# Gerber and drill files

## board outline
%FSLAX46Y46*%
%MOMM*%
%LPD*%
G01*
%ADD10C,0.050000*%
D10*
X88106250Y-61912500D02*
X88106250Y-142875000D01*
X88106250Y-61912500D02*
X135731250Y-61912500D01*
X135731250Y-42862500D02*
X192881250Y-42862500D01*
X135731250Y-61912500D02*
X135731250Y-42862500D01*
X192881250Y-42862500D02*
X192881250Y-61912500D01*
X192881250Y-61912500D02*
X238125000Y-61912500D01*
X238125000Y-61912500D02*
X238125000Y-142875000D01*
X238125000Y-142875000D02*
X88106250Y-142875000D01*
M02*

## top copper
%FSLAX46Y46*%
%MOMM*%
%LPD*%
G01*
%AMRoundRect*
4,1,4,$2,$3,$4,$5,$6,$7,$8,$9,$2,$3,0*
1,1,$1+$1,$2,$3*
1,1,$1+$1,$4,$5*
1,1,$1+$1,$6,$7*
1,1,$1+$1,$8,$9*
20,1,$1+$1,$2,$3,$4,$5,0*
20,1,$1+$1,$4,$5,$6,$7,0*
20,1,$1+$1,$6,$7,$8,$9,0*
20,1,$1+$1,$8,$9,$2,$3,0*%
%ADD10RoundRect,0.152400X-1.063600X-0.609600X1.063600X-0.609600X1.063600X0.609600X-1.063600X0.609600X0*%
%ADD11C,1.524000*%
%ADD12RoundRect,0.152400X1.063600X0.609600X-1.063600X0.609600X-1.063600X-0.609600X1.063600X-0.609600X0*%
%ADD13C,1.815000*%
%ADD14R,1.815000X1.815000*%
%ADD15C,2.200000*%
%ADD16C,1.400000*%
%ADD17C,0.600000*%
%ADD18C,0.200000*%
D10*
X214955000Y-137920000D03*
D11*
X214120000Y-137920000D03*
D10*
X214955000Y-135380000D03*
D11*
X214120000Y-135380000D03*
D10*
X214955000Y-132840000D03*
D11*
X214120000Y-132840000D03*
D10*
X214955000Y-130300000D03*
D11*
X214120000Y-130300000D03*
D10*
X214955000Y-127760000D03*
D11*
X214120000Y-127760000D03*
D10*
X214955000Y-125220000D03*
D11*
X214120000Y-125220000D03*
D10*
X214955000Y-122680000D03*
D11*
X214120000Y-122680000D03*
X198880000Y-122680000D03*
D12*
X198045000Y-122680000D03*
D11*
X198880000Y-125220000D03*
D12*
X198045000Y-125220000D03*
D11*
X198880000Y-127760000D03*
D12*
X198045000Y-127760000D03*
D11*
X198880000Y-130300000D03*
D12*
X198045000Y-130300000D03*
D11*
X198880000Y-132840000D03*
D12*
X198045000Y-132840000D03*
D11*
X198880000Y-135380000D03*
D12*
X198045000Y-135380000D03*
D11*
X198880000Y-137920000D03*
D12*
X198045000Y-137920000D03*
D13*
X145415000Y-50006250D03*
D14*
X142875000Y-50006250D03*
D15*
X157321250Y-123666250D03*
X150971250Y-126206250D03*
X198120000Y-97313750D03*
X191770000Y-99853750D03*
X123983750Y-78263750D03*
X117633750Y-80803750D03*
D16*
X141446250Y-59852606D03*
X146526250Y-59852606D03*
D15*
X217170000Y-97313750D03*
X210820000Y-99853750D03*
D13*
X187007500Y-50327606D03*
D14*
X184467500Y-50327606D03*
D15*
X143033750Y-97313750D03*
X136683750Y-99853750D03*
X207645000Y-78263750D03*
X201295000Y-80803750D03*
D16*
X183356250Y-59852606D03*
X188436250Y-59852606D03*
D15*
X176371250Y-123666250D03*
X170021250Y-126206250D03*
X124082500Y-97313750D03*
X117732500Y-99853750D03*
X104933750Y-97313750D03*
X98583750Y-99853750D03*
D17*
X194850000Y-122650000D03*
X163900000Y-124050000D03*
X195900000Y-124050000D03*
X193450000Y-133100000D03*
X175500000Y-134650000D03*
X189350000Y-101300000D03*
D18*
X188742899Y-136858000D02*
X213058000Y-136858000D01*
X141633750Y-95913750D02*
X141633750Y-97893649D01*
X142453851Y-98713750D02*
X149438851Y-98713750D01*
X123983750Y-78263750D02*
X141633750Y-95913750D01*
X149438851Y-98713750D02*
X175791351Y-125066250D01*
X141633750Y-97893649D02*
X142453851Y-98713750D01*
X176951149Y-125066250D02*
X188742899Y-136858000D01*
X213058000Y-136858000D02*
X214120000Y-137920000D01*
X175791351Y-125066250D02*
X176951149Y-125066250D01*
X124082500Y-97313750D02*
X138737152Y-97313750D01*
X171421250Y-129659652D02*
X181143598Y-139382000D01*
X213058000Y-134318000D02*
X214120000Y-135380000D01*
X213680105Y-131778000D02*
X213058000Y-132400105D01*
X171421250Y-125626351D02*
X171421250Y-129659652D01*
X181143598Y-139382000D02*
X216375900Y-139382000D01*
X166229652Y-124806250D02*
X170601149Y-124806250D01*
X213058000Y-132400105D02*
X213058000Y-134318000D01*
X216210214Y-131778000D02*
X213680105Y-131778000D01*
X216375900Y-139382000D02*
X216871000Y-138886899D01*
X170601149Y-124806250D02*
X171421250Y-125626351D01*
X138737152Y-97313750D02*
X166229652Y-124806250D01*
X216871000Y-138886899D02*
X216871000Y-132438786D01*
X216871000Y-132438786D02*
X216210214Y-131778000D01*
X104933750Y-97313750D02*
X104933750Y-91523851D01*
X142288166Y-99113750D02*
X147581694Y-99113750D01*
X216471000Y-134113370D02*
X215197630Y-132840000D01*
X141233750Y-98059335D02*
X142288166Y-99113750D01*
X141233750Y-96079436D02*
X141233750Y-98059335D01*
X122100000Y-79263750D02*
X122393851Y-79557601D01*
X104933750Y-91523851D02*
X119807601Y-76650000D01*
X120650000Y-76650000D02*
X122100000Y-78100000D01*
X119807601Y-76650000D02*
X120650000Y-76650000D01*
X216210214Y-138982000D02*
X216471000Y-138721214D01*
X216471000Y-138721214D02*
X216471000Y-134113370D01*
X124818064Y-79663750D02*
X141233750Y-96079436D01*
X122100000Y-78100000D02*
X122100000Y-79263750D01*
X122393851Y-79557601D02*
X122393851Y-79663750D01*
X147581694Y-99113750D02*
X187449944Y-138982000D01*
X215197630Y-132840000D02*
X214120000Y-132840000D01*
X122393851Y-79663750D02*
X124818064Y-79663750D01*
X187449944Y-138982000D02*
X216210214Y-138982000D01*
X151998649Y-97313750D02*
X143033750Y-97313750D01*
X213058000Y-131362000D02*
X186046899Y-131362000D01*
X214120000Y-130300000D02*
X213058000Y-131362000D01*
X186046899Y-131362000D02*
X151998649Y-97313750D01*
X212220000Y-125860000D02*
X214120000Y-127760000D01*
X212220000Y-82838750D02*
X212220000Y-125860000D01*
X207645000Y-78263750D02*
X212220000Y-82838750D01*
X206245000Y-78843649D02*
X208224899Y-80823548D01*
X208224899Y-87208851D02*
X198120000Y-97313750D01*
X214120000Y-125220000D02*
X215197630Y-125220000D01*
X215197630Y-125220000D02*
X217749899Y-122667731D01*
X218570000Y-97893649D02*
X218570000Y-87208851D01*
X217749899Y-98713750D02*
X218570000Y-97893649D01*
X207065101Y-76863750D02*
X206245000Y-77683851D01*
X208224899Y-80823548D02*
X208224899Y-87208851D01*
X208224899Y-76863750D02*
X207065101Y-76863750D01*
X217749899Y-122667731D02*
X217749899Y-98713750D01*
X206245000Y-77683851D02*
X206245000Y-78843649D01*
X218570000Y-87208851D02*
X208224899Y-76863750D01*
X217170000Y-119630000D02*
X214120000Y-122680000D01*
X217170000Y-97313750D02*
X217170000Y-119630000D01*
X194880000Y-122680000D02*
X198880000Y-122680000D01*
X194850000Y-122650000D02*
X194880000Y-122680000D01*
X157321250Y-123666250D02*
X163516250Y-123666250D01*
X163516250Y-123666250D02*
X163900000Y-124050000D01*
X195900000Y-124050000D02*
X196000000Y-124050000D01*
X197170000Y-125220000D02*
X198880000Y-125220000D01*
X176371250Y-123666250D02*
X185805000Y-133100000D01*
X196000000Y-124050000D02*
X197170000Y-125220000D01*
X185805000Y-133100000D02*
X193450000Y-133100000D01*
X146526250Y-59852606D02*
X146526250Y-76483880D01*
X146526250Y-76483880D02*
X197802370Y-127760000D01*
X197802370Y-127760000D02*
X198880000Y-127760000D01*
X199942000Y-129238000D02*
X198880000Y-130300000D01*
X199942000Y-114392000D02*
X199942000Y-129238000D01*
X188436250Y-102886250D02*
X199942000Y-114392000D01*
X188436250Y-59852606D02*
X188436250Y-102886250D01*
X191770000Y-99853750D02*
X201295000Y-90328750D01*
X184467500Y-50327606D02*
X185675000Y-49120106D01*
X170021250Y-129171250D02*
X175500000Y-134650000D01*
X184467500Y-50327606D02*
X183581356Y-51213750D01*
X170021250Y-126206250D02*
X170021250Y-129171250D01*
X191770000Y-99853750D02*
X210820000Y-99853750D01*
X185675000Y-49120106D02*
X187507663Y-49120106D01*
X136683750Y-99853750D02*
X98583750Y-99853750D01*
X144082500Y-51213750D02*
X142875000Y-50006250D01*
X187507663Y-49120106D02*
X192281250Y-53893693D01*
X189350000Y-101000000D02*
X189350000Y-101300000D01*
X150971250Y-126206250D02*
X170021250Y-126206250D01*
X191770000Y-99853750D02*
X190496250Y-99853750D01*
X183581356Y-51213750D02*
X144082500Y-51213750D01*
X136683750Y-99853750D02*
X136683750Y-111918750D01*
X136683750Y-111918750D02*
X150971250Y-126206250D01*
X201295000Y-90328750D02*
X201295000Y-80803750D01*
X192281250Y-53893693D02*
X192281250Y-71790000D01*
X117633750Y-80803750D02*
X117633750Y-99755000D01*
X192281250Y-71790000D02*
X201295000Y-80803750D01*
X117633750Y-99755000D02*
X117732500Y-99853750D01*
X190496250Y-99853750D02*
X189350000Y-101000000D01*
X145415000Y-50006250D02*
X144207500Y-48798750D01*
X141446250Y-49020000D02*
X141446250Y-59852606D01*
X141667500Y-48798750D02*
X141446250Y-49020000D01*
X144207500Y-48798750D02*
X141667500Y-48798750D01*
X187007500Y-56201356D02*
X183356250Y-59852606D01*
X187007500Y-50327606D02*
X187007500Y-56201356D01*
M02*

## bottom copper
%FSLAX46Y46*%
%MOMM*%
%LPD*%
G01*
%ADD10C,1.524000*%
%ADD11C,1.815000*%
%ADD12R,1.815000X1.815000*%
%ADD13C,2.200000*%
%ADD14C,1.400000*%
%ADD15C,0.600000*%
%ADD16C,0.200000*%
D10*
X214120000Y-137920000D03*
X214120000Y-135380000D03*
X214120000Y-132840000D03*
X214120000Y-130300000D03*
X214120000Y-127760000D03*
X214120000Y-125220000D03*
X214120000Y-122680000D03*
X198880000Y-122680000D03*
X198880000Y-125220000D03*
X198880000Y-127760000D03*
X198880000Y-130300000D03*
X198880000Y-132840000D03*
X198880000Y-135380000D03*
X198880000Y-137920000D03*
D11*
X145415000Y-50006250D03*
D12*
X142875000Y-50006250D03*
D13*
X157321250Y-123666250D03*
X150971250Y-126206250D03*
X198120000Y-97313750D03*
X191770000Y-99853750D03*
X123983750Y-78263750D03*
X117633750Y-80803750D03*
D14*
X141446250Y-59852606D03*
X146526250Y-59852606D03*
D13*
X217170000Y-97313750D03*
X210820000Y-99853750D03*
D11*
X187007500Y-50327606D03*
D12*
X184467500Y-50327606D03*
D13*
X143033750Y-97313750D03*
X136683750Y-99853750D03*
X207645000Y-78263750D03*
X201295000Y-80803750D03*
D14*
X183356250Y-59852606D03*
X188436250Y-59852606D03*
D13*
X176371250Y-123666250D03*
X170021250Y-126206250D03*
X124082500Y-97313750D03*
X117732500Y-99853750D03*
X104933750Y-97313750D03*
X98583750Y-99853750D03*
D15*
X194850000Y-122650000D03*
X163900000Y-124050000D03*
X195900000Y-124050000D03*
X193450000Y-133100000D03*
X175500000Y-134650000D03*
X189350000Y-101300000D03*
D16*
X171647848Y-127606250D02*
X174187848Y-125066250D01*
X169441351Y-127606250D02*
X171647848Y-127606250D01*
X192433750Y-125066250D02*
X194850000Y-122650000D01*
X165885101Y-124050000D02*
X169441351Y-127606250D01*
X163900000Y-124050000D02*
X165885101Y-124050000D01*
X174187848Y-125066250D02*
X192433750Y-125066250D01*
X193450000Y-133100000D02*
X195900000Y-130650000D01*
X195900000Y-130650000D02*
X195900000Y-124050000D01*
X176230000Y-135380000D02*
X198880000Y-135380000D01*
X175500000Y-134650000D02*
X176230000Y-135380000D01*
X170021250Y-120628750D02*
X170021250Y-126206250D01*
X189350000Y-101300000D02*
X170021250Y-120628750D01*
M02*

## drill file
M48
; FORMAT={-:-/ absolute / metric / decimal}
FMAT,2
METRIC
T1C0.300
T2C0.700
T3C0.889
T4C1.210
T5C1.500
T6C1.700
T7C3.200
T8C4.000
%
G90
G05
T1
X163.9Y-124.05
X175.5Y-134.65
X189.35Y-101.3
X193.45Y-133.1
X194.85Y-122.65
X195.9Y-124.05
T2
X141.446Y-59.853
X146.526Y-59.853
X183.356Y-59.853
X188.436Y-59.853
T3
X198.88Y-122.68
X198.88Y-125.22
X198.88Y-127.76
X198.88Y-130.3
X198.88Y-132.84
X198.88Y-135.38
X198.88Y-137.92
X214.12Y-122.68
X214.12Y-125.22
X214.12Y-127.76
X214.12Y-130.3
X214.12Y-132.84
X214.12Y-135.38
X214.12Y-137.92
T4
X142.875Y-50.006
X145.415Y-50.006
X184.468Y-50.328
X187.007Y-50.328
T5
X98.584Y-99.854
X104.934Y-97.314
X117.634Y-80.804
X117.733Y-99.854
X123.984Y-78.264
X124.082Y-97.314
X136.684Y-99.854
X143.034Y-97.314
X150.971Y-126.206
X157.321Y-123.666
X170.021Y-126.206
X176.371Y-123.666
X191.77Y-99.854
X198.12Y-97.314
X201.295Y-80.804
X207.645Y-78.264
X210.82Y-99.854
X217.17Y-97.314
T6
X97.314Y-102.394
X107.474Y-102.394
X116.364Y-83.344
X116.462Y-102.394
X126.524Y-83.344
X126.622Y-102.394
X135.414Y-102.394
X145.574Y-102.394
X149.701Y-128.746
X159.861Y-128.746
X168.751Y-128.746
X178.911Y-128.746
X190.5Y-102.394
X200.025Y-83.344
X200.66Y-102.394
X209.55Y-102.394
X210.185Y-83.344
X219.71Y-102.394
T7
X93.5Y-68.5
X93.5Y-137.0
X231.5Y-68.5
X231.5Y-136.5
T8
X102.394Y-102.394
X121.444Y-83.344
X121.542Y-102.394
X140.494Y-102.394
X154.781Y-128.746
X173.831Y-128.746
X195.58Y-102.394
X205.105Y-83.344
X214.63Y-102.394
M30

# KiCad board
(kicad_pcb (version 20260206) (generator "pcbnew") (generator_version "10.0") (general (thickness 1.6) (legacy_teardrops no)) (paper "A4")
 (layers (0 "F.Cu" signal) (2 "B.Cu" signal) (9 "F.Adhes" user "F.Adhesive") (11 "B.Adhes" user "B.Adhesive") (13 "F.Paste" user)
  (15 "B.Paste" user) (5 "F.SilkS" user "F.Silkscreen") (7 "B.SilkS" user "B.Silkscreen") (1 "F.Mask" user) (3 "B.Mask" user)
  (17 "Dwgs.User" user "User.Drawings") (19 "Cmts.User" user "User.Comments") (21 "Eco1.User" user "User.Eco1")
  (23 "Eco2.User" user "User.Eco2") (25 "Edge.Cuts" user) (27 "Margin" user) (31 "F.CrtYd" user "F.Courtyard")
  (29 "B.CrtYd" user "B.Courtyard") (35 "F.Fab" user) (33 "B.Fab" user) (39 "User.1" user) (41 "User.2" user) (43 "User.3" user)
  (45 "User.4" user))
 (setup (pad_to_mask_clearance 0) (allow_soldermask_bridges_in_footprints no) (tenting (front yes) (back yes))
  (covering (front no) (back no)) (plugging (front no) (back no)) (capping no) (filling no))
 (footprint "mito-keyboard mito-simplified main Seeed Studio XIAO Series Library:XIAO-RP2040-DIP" (layer "F.Cu") (at 206.5 130.3 180)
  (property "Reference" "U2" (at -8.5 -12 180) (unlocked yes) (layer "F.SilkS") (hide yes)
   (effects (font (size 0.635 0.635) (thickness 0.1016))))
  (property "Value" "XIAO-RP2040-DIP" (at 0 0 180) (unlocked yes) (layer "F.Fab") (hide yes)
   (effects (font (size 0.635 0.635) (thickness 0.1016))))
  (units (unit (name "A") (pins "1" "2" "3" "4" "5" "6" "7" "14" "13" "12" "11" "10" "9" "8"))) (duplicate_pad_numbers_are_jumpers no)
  (pad "1" smd roundrect (at -8.455 -7.62) (size 2.432 1.524) (layers "F.Cu" "F.Mask") (roundrect_rratio 0.1) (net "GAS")
   (thermal_bridge_angle 45))
  (pad "1" thru_hole circle (at -7.62 -7.62) (size 1.524 1.524) (drill 0.889) (layers "*.Cu" "*.Mask") (remove_unused_layers no) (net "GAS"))
  (pad "2" smd roundrect (at -8.455 -5.08) (size 2.432 1.524) (layers "F.Cu" "F.Mask") (roundrect_rratio 0.1) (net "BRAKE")
   (thermal_bridge_angle 45))
  (pad "2" thru_hole circle (at -7.62 -5.08) (size 1.524 1.524) (drill 0.889) (layers "*.Cu" "*.Mask") (remove_unused_layers no)
   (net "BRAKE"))
  (pad "3" smd roundrect (at -8.455 -2.54) (size 2.432 1.524) (layers "F.Cu" "F.Mask") (roundrect_rratio 0.1) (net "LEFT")
   (thermal_bridge_angle 45))
  (pad "3" thru_hole circle (at -7.62 -2.54) (size 1.524 1.524) (drill 0.889) (layers "*.Cu" "*.Mask") (remove_unused_layers no)
   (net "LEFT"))
  (pad "4" smd roundrect (at -8.455 0) (size 2.432 1.524) (layers "F.Cu" "F.Mask") (roundrect_rratio 0.1) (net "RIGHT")
   (thermal_bridge_angle 45))
  (pad "4" thru_hole circle (at -7.62 0) (size 1.524 1.524) (drill 0.889) (layers "*.Cu" "*.Mask") (remove_unused_layers no) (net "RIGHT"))
  (pad "5" smd roundrect (at -8.455 2.54) (size 2.432 1.524) (layers "F.Cu" "F.Mask") (roundrect_rratio 0.1) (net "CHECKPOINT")
   (thermal_bridge_angle 45))
  (pad "5" thru_hole circle (at -7.62 2.54) (size 1.524 1.524) (drill 0.889) (layers "*.Cu" "*.Mask") (remove_unused_layers no)
   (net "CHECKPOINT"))
  (pad "6" smd roundrect (at -8.455 5.08) (size 2.432 1.524) (layers "F.Cu" "F.Mask") (roundrect_rratio 0.1) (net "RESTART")
   (thermal_bridge_angle 45))
  (pad "6" thru_hole circle (at -7.62 5.08) (size 1.524 1.524) (drill 0.889) (layers "*.Cu" "*.Mask") (remove_unused_layers no)
   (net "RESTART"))
  (pad "7" smd roundrect (at -8.455 7.62) (size 2.432 1.524) (layers "F.Cu" "F.Mask") (roundrect_rratio 0.1) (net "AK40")
   (thermal_bridge_angle 45))
  (pad "7" thru_hole circle (at -7.62 7.62) (size 1.524 1.524) (drill 0.889) (layers "*.Cu" "*.Mask") (remove_unused_layers no) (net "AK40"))
  (pad "8" thru_hole circle (at 7.62 7.62 180) (size 1.524 1.524) (drill 0.889) (layers "*.Cu" "*.Mask") (remove_unused_layers no)
   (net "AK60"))
  (pad "8" smd roundrect (at 8.455 7.62 180) (size 2.432 1.524) (layers "F.Cu" "F.Mask") (roundrect_rratio 0.1) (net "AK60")
   (thermal_bridge_angle 45))
  (pad "9" thru_hole circle (at 7.62 5.08 180) (size 1.524 1.524) (drill 0.889) (layers "*.Cu" "*.Mask") (remove_unused_layers no)
   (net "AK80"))
  (pad "9" smd roundrect (at 8.455 5.08 180) (size 2.432 1.524) (layers "F.Cu" "F.Mask") (roundrect_rratio 0.1) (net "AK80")
   (thermal_bridge_angle 45))
  (pad "10" thru_hole circle (at 7.62 2.54 180) (size 1.524 1.524) (drill 0.889) (layers "*.Cu" "*.Mask") (remove_unused_layers no)
   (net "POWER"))
  (pad "10" smd roundrect (at 8.455 2.54 180) (size 2.432 1.524) (layers "F.Cu" "F.Mask") (roundrect_rratio 0.1) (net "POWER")
   (thermal_bridge_angle 45))
  (pad "11" thru_hole circle (at 7.62 0 180) (size 1.524 1.524) (drill 0.889) (layers "*.Cu" "*.Mask") (remove_unused_layers no)
   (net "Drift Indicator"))
  (pad "11" smd roundrect (at 8.455 0 180) (size 2.432 1.524) (layers "F.Cu" "F.Mask") (roundrect_rratio 0.1) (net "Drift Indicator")
   (thermal_bridge_angle 45))
  (pad "12" thru_hole circle (at 7.62 -2.54 180) (size 1.524 1.524) (drill 0.889) (layers "*.Cu" "*.Mask") (remove_unused_layers no)
   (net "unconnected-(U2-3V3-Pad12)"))
  (pad "12" smd roundrect (at 8.455 -2.54 180) (size 2.432 1.524) (layers "F.Cu" "F.Mask") (roundrect_rratio 0.1)
   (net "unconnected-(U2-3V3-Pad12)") (thermal_bridge_angle 45))
  (pad "13" thru_hole circle (at 7.62 -5.08 180) (size 1.524 1.524) (drill 0.889) (layers "*.Cu" "*.Mask") (remove_unused_layers no)
   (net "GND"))
  (pad "13" smd roundrect (at 8.455 -5.08 180) (size 2.432 1.524) (layers "F.Cu" "F.Mask") (roundrect_rratio 0.1) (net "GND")
   (thermal_bridge_angle 45))
  (pad "14" thru_hole circle (at 7.62 -7.62 180) (size 1.524 1.524) (drill 0.889) (layers "*.Cu" "*.Mask") (remove_unused_layers no)
   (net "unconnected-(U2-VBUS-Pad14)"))
  (pad "14" smd roundrect (at 8.455 -7.62 180) (size 2.432 1.524) (layers "F.Cu" "F.Mask") (roundrect_rratio 0.1)
   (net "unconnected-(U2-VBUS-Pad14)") (thermal_bridge_angle 45)))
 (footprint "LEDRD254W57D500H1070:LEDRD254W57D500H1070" (layer "F.Cu") (at 144.145 50.00625)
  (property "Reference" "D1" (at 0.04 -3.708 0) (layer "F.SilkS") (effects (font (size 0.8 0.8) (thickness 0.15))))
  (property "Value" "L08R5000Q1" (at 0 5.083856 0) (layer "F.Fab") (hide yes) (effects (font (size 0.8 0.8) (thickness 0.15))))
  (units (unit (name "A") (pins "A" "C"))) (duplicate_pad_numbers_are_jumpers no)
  (pad "A" thru_hole circle (at 1.27 0) (size 1.815 1.815) (drill 1.21) (layers "*.Cu" "*.Mask") (remove_unused_layers no)
   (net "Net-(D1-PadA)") (solder_mask_margin 0.102))
  (pad "C" thru_hole rect (at -1.27 0) (size 1.815 1.815) (drill 1.21) (layers "*.Cu" "*.Mask") (remove_unused_layers no) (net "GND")
   (solder_mask_margin 0.102)))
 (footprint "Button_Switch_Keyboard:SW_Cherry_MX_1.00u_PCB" (layer "F.Cu") (at 157.32125 123.66625)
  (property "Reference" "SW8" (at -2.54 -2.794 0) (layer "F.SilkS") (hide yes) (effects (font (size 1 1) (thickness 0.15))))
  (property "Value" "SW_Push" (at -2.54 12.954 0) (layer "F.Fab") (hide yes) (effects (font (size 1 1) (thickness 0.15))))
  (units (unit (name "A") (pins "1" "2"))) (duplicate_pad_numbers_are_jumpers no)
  (pad "" np_thru_hole circle (at -7.62 5.08) (size 1.7 1.7) (drill 1.7) (layers "*.Cu" "*.Mask"))
  (pad "" np_thru_hole circle (at -2.54 5.08) (size 4 4) (drill 4) (layers "*.Cu" "*.Mask"))
  (pad "" np_thru_hole circle (at 2.54 5.08) (size 1.7 1.7) (drill 1.7) (layers "*.Cu" "*.Mask"))
  (pad "1" thru_hole circle (at 0 0) (size 2.2 2.2) (drill 1.5) (layers "*.Cu" "*.Mask") (remove_unused_layers no) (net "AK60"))
  (pad "2" thru_hole circle (at -6.35 2.54) (size 2.2 2.2) (drill 1.5) (layers "*.Cu" "*.Mask") (remove_unused_layers no) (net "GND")))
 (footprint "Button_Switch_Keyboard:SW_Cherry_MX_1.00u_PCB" (layer "F.Cu") (at 198.12 97.31375)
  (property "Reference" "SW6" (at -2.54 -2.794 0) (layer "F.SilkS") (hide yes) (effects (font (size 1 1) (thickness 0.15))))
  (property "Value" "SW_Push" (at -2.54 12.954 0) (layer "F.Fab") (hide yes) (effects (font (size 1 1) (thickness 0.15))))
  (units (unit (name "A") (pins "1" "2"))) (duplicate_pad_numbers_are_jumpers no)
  (pad "" np_thru_hole circle (at -7.62 5.08) (size 1.7 1.7) (drill 1.7) (layers "*.Cu" "*.Mask"))
  (pad "" np_thru_hole circle (at -2.54 5.08) (size 4 4) (drill 4) (layers "*.Cu" "*.Mask"))
  (pad "" np_thru_hole circle (at 2.54 5.08) (size 1.7 1.7) (drill 1.7) (layers "*.Cu" "*.Mask"))
  (pad "1" thru_hole circle (at 0 0) (size 2.2 2.2) (drill 1.5) (layers "*.Cu" "*.Mask") (remove_unused_layers no) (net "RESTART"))
  (pad "2" thru_hole circle (at -6.35 2.54) (size 2.2 2.2) (drill 1.5) (layers "*.Cu" "*.Mask") (remove_unused_layers no) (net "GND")))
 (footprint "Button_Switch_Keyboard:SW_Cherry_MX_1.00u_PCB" (layer "F.Cu") (at 123.98375 78.26375)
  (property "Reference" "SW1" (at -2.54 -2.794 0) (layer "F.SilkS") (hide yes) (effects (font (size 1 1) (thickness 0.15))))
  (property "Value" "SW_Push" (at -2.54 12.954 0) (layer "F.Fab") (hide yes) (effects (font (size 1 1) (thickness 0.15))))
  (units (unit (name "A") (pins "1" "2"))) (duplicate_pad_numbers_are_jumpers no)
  (pad "" np_thru_hole circle (at -7.62 5.08) (size 1.7 1.7) (drill 1.7) (layers "*.Cu" "*.Mask"))
  (pad "" np_thru_hole circle (at -2.54 5.08) (size 4 4) (drill 4) (layers "*.Cu" "*.Mask"))
  (pad "" np_thru_hole circle (at 2.54 5.08) (size 1.7 1.7) (drill 1.7) (layers "*.Cu" "*.Mask"))
  (pad "1" thru_hole circle (at 0 0) (size 2.2 2.2) (drill 1.5) (layers "*.Cu" "*.Mask") (remove_unused_layers no) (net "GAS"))
  (pad "2" thru_hole circle (at -6.35 2.54) (size 2.2 2.2) (drill 1.5) (layers "*.Cu" "*.Mask") (remove_unused_layers no) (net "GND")))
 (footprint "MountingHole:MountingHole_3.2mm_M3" (layer "F.Cu") (at 93.5 68.5)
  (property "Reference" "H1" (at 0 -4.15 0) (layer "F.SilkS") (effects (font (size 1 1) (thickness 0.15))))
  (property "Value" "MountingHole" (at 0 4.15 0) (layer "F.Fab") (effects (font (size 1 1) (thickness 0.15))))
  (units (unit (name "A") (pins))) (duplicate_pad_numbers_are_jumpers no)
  (pad "" np_thru_hole circle (at 0 0) (size 3.2 3.2) (drill 3.2) (layers "*.Cu" "*.Mask")))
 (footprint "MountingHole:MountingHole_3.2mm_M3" (layer "F.Cu") (at 93.5 137)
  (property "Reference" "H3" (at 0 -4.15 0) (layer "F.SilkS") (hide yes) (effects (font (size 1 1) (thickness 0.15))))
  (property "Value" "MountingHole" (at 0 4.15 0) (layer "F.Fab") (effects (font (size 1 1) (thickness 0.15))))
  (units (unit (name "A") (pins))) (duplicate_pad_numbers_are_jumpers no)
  (pad "" np_thru_hole circle (at 0 0) (size 3.2 3.2) (drill 3.2) (layers "*.Cu" "*.Mask")))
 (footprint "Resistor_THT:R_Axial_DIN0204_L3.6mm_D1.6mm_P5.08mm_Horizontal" (layer "F.Cu") (at 141.44625 59.852606)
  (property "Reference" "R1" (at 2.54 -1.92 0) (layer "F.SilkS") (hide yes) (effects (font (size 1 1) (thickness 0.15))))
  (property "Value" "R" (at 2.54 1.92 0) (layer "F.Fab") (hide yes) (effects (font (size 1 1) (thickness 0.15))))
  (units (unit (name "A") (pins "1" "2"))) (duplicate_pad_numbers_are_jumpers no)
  (pad "1" thru_hole circle (at 0 0) (size 1.4 1.4) (drill 0.7) (layers "*.Cu" "*.Mask") (remove_unused_layers no) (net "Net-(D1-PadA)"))
  (pad "2" thru_hole circle (at 5.08 0) (size 1.4 1.4) (drill 0.7) (layers "*.Cu" "*.Mask") (remove_unused_layers no) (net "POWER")))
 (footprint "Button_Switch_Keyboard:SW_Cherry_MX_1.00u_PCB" (layer "F.Cu") (at 217.17 97.31375)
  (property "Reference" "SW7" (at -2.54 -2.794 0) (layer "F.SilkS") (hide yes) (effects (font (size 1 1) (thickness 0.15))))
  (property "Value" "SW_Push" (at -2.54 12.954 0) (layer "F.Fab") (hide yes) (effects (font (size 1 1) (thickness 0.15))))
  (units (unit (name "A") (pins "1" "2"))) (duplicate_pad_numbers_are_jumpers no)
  (pad "" np_thru_hole circle (at -7.62 5.08) (size 1.7 1.7) (drill 1.7) (layers "*.Cu" "*.Mask"))
  (pad "" np_thru_hole circle (at -2.54 5.08) (size 4 4) (drill 4) (layers "*.Cu" "*.Mask"))
  (pad "" np_thru_hole circle (at 2.54 5.08) (size 1.7 1.7) (drill 1.7) (layers "*.Cu" "*.Mask"))
  (pad "1" thru_hole circle (at 0 0) (size 2.2 2.2) (drill 1.5) (layers "*.Cu" "*.Mask") (remove_unused_layers no) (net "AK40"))
  (pad "2" thru_hole circle (at -6.35 2.54) (size 2.2 2.2) (drill 1.5) (layers "*.Cu" "*.Mask") (remove_unused_layers no) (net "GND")))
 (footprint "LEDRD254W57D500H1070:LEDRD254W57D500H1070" (layer "F.Cu") (at 185.7375 50.327606)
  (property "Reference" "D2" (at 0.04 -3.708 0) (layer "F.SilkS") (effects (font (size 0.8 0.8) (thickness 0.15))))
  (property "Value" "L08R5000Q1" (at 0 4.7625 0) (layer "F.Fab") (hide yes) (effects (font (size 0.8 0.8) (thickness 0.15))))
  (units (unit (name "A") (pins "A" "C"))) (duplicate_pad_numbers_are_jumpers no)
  (pad "A" thru_hole circle (at 1.27 0) (size 1.815 1.815) (drill 1.21) (layers "*.Cu" "*.Mask") (remove_unused_layers no)
   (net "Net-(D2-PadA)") (solder_mask_margin 0.102))
  (pad "C" thru_hole rect (at -1.27 0) (size 1.815 1.815) (drill 1.21) (layers "*.Cu" "*.Mask") (remove_unused_layers no) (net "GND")
   (solder_mask_margin 0.102)))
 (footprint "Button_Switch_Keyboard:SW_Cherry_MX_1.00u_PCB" (layer "F.Cu") (at 143.03375 97.31375)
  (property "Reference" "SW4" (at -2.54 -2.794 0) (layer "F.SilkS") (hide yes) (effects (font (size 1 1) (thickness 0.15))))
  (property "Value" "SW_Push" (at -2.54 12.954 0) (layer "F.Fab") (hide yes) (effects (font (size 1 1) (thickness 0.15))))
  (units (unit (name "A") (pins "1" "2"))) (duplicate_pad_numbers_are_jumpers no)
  (pad "" np_thru_hole circle (at -7.62 5.08) (size 1.7 1.7) (drill 1.7) (layers "*.Cu" "*.Mask"))
  (pad "" np_thru_hole circle (at -2.54 5.08) (size 4 4) (drill 4) (layers "*.Cu" "*.Mask"))
  (pad "" np_thru_hole circle (at 2.54 5.08) (size 1.7 1.7) (drill 1.7) (layers "*.Cu" "*.Mask"))
  (pad "1" thru_hole circle (at 0 0) (size 2.2 2.2) (drill 1.5) (layers "*.Cu" "*.Mask") (remove_unused_layers no) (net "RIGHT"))
  (pad "2" thru_hole circle (at -6.35 2.54) (size 2.2 2.2) (drill 1.5) (layers "*.Cu" "*.Mask") (remove_unused_layers no) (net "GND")))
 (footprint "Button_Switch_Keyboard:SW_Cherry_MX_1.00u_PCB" (layer "F.Cu") (at 207.645 78.26375)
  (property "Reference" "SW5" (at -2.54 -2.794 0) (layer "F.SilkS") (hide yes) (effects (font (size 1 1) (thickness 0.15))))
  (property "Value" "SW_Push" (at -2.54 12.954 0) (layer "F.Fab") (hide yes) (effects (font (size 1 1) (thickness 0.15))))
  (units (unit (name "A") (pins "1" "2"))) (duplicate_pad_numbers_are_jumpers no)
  (pad "" np_thru_hole circle (at -7.62 5.08) (size 1.7 1.7) (drill 1.7) (layers "*.Cu" "*.Mask"))
  (pad "" np_thru_hole circle (at -2.54 5.08) (size 4 4) (drill 4) (layers "*.Cu" "*.Mask"))
  (pad "" np_thru_hole circle (at 2.54 5.08) (size 1.7 1.7) (drill 1.7) (layers "*.Cu" "*.Mask"))
  (pad "1" thru_hole circle (at 0 0) (size 2.2 2.2) (drill 1.5) (layers "*.Cu" "*.Mask") (remove_unused_layers no) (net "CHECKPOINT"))
  (pad "2" thru_hole circle (at -6.35 2.54) (size 2.2 2.2) (drill 1.5) (layers "*.Cu" "*.Mask") (remove_unused_layers no) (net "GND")))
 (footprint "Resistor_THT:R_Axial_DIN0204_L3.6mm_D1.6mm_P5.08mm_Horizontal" (layer "F.Cu") (at 183.35625 59.852606)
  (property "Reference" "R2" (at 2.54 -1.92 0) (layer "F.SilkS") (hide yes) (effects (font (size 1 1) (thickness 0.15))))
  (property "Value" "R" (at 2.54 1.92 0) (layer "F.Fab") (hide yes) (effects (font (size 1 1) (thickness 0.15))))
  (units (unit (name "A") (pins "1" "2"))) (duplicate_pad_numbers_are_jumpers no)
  (pad "1" thru_hole circle (at 0 0) (size 1.4 1.4) (drill 0.7) (layers "*.Cu" "*.Mask") (remove_unused_layers no) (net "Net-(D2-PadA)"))
  (pad "2" thru_hole circle (at 5.08 0) (size 1.4 1.4) (drill 0.7) (layers "*.Cu" "*.Mask") (remove_unused_layers no)
   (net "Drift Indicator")))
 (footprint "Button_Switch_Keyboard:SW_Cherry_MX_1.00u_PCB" (layer "F.Cu") (at 176.37125 123.66625)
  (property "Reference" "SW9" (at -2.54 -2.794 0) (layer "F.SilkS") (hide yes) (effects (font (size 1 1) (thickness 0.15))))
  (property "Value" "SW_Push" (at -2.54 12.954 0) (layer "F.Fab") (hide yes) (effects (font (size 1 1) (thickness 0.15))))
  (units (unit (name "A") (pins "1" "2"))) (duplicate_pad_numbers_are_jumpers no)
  (pad "" np_thru_hole circle (at -7.62 5.08) (size 1.7 1.7) (drill 1.7) (layers "*.Cu" "*.Mask"))
  (pad "" np_thru_hole circle (at -2.54 5.08) (size 4 4) (drill 4) (layers "*.Cu" "*.Mask"))
  (pad "" np_thru_hole circle (at 2.54 5.08) (size 1.7 1.7) (drill 1.7) (layers "*.Cu" "*.Mask"))
  (pad "1" thru_hole circle (at 0 0) (size 2.2 2.2) (drill 1.5) (layers "*.Cu" "*.Mask") (remove_unused_layers no) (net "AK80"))
  (pad "2" thru_hole circle (at -6.35 2.54) (size 2.2 2.2) (drill 1.5) (layers "*.Cu" "*.Mask") (remove_unused_layers no) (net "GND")))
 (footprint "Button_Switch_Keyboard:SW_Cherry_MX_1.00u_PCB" (layer "F.Cu") (at 124.0825 97.31375)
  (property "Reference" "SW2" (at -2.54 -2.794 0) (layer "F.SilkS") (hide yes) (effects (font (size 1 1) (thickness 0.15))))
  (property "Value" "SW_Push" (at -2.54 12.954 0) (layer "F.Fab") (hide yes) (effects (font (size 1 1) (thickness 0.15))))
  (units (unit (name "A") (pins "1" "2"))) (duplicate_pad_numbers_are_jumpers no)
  (pad "" np_thru_hole circle (at -7.62 5.08) (size 1.7 1.7) (drill 1.7) (layers "*.Cu" "*.Mask"))
  (pad "" np_thru_hole circle (at -2.54 5.08) (size 4 4) (drill 4) (layers "*.Cu" "*.Mask"))
  (pad "" np_thru_hole circle (at 2.54 5.08) (size 1.7 1.7) (drill 1.7) (layers "*.Cu" "*.Mask"))
  (pad "1" thru_hole circle (at 0 0) (size 2.2 2.2) (drill 1.5) (layers "*.Cu" "*.Mask") (remove_unused_layers no) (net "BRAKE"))
  (pad "2" thru_hole circle (at -6.35 2.54) (size 2.2 2.2) (drill 1.5) (layers "*.Cu" "*.Mask") (remove_unused_layers no) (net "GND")))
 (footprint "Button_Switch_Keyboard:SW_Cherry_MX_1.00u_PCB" (layer "F.Cu") (at 104.93375 97.31375)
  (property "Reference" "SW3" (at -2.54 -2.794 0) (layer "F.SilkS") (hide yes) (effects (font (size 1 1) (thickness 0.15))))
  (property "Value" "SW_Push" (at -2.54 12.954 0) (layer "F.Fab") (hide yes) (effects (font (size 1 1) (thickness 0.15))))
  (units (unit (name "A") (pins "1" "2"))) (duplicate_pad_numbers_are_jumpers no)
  (pad "" np_thru_hole circle (at -7.62 5.08) (size 1.7 1.7) (drill 1.7) (layers "*.Cu" "*.Mask"))
  (pad "" np_thru_hole circle (at -2.54 5.08) (size 4 4) (drill 4) (layers "*.Cu" "*.Mask"))
  (pad "" np_thru_hole circle (at 2.54 5.08) (size 1.7 1.7) (drill 1.7) (layers "*.Cu" "*.Mask"))
  (pad "1" thru_hole circle (at 0 0) (size 2.2 2.2) (drill 1.5) (layers "*.Cu" "*.Mask") (remove_unused_layers no) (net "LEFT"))
  (pad "2" thru_hole circle (at -6.35 2.54) (size 2.2 2.2) (drill 1.5) (layers "*.Cu" "*.Mask") (remove_unused_layers no) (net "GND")))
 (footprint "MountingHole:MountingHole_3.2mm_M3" (layer "F.Cu") (at 231.5 68.5)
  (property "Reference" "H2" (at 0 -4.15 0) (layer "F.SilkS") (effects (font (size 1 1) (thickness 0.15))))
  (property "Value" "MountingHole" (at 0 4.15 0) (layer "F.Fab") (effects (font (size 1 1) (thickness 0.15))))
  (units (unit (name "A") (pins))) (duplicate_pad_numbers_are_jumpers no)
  (pad "" np_thru_hole circle (at 0 0) (size 3.2 3.2) (drill 3.2) (layers "*.Cu" "*.Mask")))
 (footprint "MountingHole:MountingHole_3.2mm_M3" (layer "F.Cu") (at 231.5 136.5)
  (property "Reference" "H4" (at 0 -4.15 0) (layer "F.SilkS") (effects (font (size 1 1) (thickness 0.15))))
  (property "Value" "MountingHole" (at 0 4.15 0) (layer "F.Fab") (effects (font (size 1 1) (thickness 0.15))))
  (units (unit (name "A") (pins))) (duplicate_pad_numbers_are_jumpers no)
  (pad "" np_thru_hole circle (at 0 0) (size 3.2 3.2) (drill 3.2) (layers "*.Cu" "*.Mask")))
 (gr_line (start 88.10625 61.9125) (end 88.10625 142.875) (stroke (width 0.05) (type default)) (layer "Edge.Cuts"))
 (gr_line (start 88.10625 61.9125) (end 135.73125 61.9125) (stroke (width 0.05) (type default)) (layer "Edge.Cuts"))
 (gr_line (start 135.73125 42.8625) (end 192.88125 42.8625) (stroke (width 0.05) (type default)) (layer "Edge.Cuts"))
 (gr_line (start 135.73125 61.9125) (end 135.73125 42.8625) (stroke (width 0.05) (type default)) (layer "Edge.Cuts"))
 (gr_line (start 192.88125 42.8625) (end 192.88125 61.9125) (stroke (width 0.05) (type default)) (layer "Edge.Cuts"))
 (gr_line (start 192.88125 61.9125) (end 238.125 61.9125) (stroke (width 0.05) (type default)) (layer "Edge.Cuts"))
 (gr_line (start 238.125 61.9125) (end 238.125 142.875) (stroke (width 0.05) (type default)) (layer "Edge.Cuts"))
 (gr_line (start 238.125 142.875) (end 88.10625 142.875) (stroke (width 0.05) (type default)) (layer "Edge.Cuts"))
 (segment (start 188.742899 136.858) (end 213.058 136.858) (width 0.2) (layer "F.Cu") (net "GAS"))
 (segment (start 141.63375 95.91375) (end 141.63375 97.893649) (width 0.2) (layer "F.Cu") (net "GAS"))
 (segment (start 142.453851 98.71375) (end 149.438851 98.71375) (width 0.2) (layer "F.Cu") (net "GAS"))
 (segment (start 123.98375 78.26375) (end 141.63375 95.91375) (width 0.2) (layer "F.Cu") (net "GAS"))
 (segment (start 149.438851 98.71375) (end 175.791351 125.06625) (width 0.2) (layer "F.Cu") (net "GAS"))
 (segment (start 141.63375 97.893649) (end 142.453851 98.71375) (width 0.2) (layer "F.Cu") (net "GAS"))
 (segment (start 176.951149 125.06625) (end 188.742899 136.858) (width 0.2) (layer "F.Cu") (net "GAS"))
 (segment (start 213.058 136.858) (end 214.12 137.92) (width 0.2) (layer "F.Cu") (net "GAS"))
 (segment (start 175.791351 125.06625) (end 176.951149 125.06625) (width 0.2) (layer "F.Cu") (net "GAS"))
 (segment (start 124.0825 97.31375) (end 138.737152 97.31375) (width 0.2) (layer "F.Cu") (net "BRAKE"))
 (segment (start 171.42125 129.659652) (end 181.143598 139.382) (width 0.2) (layer "F.Cu") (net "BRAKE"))
 (segment (start 213.058 134.318) (end 214.12 135.38) (width 0.2) (layer "F.Cu") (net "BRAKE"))
 (segment (start 213.680105 131.778) (end 213.058 132.400105) (width 0.2) (layer "F.Cu") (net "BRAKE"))
 (segment (start 171.42125 125.626351) (end 171.42125 129.659652) (width 0.2) (layer "F.Cu") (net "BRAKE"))
 (segment (start 181.143598 139.382) (end 216.3759 139.382) (width 0.2) (layer "F.Cu") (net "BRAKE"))
 (segment (start 166.229652 124.80625) (end 170.601149 124.80625) (width 0.2) (layer "F.Cu") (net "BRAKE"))
 (segment (start 213.058 132.400105) (end 213.058 134.318) (width 0.2) (layer "F.Cu") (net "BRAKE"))
 (segment (start 216.210214 131.778) (end 213.680105 131.778) (width 0.2) (layer "F.Cu") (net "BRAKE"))
 (segment (start 216.3759 139.382) (end 216.871 138.886899) (width 0.2) (layer "F.Cu") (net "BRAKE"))
 (segment (start 170.601149 124.80625) (end 171.42125 125.626351) (width 0.2) (layer "F.Cu") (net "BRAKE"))
 (segment (start 138.737152 97.31375) (end 166.229652 124.80625) (width 0.2) (layer "F.Cu") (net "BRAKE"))
 (segment (start 216.871 138.886899) (end 216.871 132.438786) (width 0.2) (layer "F.Cu") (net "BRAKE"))
 (segment (start 216.871 132.438786) (end 216.210214 131.778) (width 0.2) (layer "F.Cu") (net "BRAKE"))
 (segment (start 104.93375 97.31375) (end 104.93375 91.523851) (width 0.2) (layer "F.Cu") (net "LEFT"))
 (segment (start 142.288166 99.11375) (end 147.581694 99.11375) (width 0.2) (layer "F.Cu") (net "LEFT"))
 (segment (start 216.471 134.11337) (end 215.19763 132.84) (width 0.2) (layer "F.Cu") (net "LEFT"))
 (segment (start 141.23375 98.059335) (end 142.288166 99.11375) (width 0.2) (layer "F.Cu") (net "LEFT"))
 (segment (start 141.23375 96.079436) (end 141.23375 98.059335) (width 0.2) (layer "F.Cu") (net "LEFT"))
 (segment (start 122.1 79.26375) (end 122.393851 79.557601) (width 0.2) (layer "F.Cu") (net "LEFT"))
 (segment (start 104.93375 91.523851) (end 119.807601 76.65) (width 0.2) (layer "F.Cu") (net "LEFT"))
 (segment (start 120.65 76.65) (end 122.1 78.1) (width 0.2) (layer "F.Cu") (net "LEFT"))
 (segment (start 119.807601 76.65) (end 120.65 76.65) (width 0.2) (layer "F.Cu") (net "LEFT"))
 (segment (start 216.210214 138.982) (end 216.471 138.721214) (width 0.2) (layer "F.Cu") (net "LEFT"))
 (segment (start 216.471 138.721214) (end 216.471 134.11337) (width 0.2) (layer "F.Cu") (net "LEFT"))
 (segment (start 124.818064 79.66375) (end 141.23375 96.079436) (width 0.2) (layer "F.Cu") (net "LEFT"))
 (segment (start 122.1 78.1) (end 122.1 79.26375) (width 0.2) (layer "F.Cu") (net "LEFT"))
 (segment (start 122.393851 79.557601) (end 122.393851 79.66375) (width 0.2) (layer "F.Cu") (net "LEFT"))
 (segment (start 147.581694 99.11375) (end 187.449944 138.982) (width 0.2) (layer "F.Cu") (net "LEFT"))
 (segment (start 215.19763 132.84) (end 214.12 132.84) (width 0.2) (layer "F.Cu") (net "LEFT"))
 (segment (start 122.393851 79.66375) (end 124.818064 79.66375) (width 0.2) (layer "F.Cu") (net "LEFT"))
 (segment (start 187.449944 138.982) (end 216.210214 138.982) (width 0.2) (layer "F.Cu") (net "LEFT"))
 (segment (start 151.998649 97.31375) (end 143.03375 97.31375) (width 0.2) (layer "F.Cu") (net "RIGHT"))
 (segment (start 213.058 131.362) (end 186.046899 131.362) (width 0.2) (layer "F.Cu") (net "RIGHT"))
 (segment (start 214.12 130.3) (end 213.058 131.362) (width 0.2) (layer "F.Cu") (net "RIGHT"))
 (segment (start 186.046899 131.362) (end 151.998649 97.31375) (width 0.2) (layer "F.Cu") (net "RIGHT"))
 (segment (start 212.22 125.86) (end 214.12 127.76) (width 0.2) (layer "F.Cu") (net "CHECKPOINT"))
 (segment (start 212.22 82.83875) (end 212.22 125.86) (width 0.2) (layer "F.Cu") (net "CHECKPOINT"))
 (segment (start 207.645 78.26375) (end 212.22 82.83875) (width 0.2) (layer "F.Cu") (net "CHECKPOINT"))
 (segment (start 206.245 78.843649) (end 208.224899 80.823548) (width 0.2) (layer "F.Cu") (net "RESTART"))
 (segment (start 208.224899 87.208851) (end 198.12 97.31375) (width 0.2) (layer "F.Cu") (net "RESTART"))
 (segment (start 214.12 125.22) (end 215.19763 125.22) (width 0.2) (layer "F.Cu") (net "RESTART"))
 (segment (start 215.19763 125.22) (end 217.749899 122.667731) (width 0.2) (layer "F.Cu") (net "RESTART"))
 (segment (start 218.57 97.893649) (end 218.57 87.208851) (width 0.2) (layer "F.Cu") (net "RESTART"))
 (segment (start 217.749899 98.71375) (end 218.57 97.893649) (width 0.2) (layer "F.Cu") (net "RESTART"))
 (segment (start 207.065101 76.86375) (end 206.245 77.683851) (width 0.2) (layer "F.Cu") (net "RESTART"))
 (segment (start 208.224899 80.823548) (end 208.224899 87.208851) (width 0.2) (layer "F.Cu") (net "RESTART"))
 (segment (start 208.224899 76.86375) (end 207.065101 76.86375) (width 0.2) (layer "F.Cu") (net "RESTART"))
 (segment (start 217.749899 122.667731) (end 217.749899 98.71375) (width 0.2) (layer "F.Cu") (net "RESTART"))
 (segment (start 206.245 77.683851) (end 206.245 78.843649) (width 0.2) (layer "F.Cu") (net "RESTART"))
 (segment (start 218.57 87.208851) (end 208.224899 76.86375) (width 0.2) (layer "F.Cu") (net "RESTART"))
 (segment (start 217.17 119.63) (end 214.12 122.68) (width 0.2) (layer "F.Cu") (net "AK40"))
 (segment (start 217.17 97.31375) (end 217.17 119.63) (width 0.2) (layer "F.Cu") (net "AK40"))
 (segment (start 194.88 122.68) (end 198.88 122.68) (width 0.2) (layer "F.Cu") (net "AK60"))
 (segment (start 194.85 122.65) (end 194.88 122.68) (width 0.2) (layer "F.Cu") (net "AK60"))
 (segment (start 157.32125 123.66625) (end 163.51625 123.66625) (width 0.2) (layer "F.Cu") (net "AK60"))
 (segment (start 163.51625 123.66625) (end 163.9 124.05) (width 0.2) (layer "F.Cu") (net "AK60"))
 (via (at 194.85 122.65) (size 0.6) (drill 0.3) (layers "F.Cu" "B.Cu") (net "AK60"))
 (via (at 163.9 124.05) (size 0.6) (drill 0.3) (layers "F.Cu" "B.Cu") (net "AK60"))
 (segment (start 171.647848 127.60625) (end 174.187848 125.06625) (width 0.2) (layer "B.Cu") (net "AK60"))
 (segment (start 169.441351 127.60625) (end 171.647848 127.60625) (width 0.2) (layer "B.Cu") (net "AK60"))
 (segment (start 192.43375 125.06625) (end 194.85 122.65) (width 0.2) (layer "B.Cu") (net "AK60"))
 (segment (start 165.885101 124.05) (end 169.441351 127.60625) (width 0.2) (layer "B.Cu") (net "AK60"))
 (segment (start 163.9 124.05) (end 165.885101 124.05) (width 0.2) (layer "B.Cu") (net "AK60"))
 (segment (start 174.187848 125.06625) (end 192.43375 125.06625) (width 0.2) (layer "B.Cu") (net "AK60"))
 (segment (start 195.9 124.05) (end 196 124.05) (width 0.2) (layer "F.Cu") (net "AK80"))
 (segment (start 197.17 125.22) (end 198.88 125.22) (width 0.2) (layer "F.Cu") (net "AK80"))
 (segment (start 176.37125 123.66625) (end 185.805 133.1) (width 0.2) (layer "F.Cu") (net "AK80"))
 (segment (start 196 124.05) (end 197.17 125.22) (width 0.2) (layer "F.Cu") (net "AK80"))
 (segment (start 185.805 133.1) (end 193.45 133.1) (width 0.2) (layer "F.Cu") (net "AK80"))
 (via (at 195.9 124.05) (size 0.6) (drill 0.3) (layers "F.Cu" "B.Cu") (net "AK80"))
 (via (at 193.45 133.1) (size 0.6) (drill 0.3) (layers "F.Cu" "B.Cu") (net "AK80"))
 (segment (start 193.45 133.1) (end 195.9 130.65) (width 0.2) (layer "B.Cu") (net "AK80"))
 (segment (start 195.9 130.65) (end 195.9 124.05) (width 0.2) (layer "B.Cu") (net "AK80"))
 (segment (start 146.52625 59.852606) (end 146.52625 76.48388) (width 0.2) (layer "F.Cu") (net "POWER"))
 (segment (start 146.52625 76.48388) (end 197.80237 127.76) (width 0.2) (layer "F.Cu") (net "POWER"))
 (segment (start 197.80237 127.76) (end 198.88 127.76) (width 0.2) (layer "F.Cu") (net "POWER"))
 (segment (start 199.942 129.238) (end 198.88 130.3) (width 0.2) (layer "F.Cu") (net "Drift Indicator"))
 (segment (start 199.942 114.392) (end 199.942 129.238) (width 0.2) (layer "F.Cu") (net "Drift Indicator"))
 (segment (start 188.43625 102.88625) (end 199.942 114.392) (width 0.2) (layer "F.Cu") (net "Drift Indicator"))
 (segment (start 188.43625 59.852606) (end 188.43625 102.88625) (width 0.2) (layer "F.Cu") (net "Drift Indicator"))
 (segment (start 191.77 99.85375) (end 201.295 90.32875) (width 0.2) (layer "F.Cu") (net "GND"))
 (segment (start 184.4675 50.327606) (end 185.675 49.120106) (width 0.2) (layer "F.Cu") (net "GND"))
 (segment (start 170.02125 129.17125) (end 175.5 134.65) (width 0.2) (layer "F.Cu") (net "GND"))
 (segment (start 184.4675 50.327606) (end 183.581356 51.21375) (width 0.2) (layer "F.Cu") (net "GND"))
 (segment (start 170.02125 126.20625) (end 170.02125 129.17125) (width 0.2) (layer "F.Cu") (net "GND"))
 (segment (start 191.77 99.85375) (end 210.82 99.85375) (width 0.2) (layer "F.Cu") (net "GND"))
 (segment (start 185.675 49.120106) (end 187.507663 49.120106) (width 0.2) (layer "F.Cu") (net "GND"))
 (segment (start 136.68375 99.85375) (end 98.58375 99.85375) (width 0.2) (layer "F.Cu") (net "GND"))
 (segment (start 144.0825 51.21375) (end 142.875 50.00625) (width 0.2) (layer "F.Cu") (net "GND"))
 (segment (start 187.507663 49.120106) (end 192.28125 53.893693) (width 0.2) (layer "F.Cu") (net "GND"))
 (segment (start 189.35 101) (end 189.35 101.3) (width 0.2) (layer "F.Cu") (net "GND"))
 (segment (start 150.97125 126.20625) (end 170.02125 126.20625) (width 0.2) (layer "F.Cu") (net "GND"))
 (segment (start 191.77 99.85375) (end 190.49625 99.85375) (width 0.2) (layer "F.Cu") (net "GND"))
 (segment (start 183.581356 51.21375) (end 144.0825 51.21375) (width 0.2) (layer "F.Cu") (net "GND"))
 (segment (start 136.68375 99.85375) (end 136.68375 111.91875) (width 0.2) (layer "F.Cu") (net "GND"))
 (segment (start 136.68375 111.91875) (end 150.97125 126.20625) (width 0.2) (layer "F.Cu") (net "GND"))
 (segment (start 201.295 90.32875) (end 201.295 80.80375) (width 0.2) (layer "F.Cu") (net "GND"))
 (segment (start 192.28125 53.893693) (end 192.28125 71.79) (width 0.2) (layer "F.Cu") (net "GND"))
 (segment (start 117.63375 80.80375) (end 117.63375 99.755) (width 0.2) (layer "F.Cu") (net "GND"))
 (segment (start 192.28125 71.79) (end 201.295 80.80375) (width 0.2) (layer "F.Cu") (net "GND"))
 (segment (start 117.63375 99.755) (end 117.7325 99.85375) (width 0.2) (layer "F.Cu") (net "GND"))
 (segment (start 190.49625 99.85375) (end 189.35 101) (width 0.2) (layer "F.Cu") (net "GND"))
 (via (at 175.5 134.65) (size 0.6) (drill 0.3) (layers "F.Cu" "B.Cu") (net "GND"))
 (via (at 189.35 101.3) (size 0.6) (drill 0.3) (layers "F.Cu" "B.Cu") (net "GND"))
 (segment (start 176.23 135.38) (end 198.88 135.38) (width 0.2) (layer "B.Cu") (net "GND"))
 (segment (start 175.5 134.65) (end 176.23 135.38) (width 0.2) (layer "B.Cu") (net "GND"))
 (segment (start 170.02125 120.62875) (end 170.02125 126.20625) (width 0.2) (layer "B.Cu") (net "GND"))
 (segment (start 189.35 101.3) (end 170.02125 120.62875) (width 0.2) (layer "B.Cu") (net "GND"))
 (segment (start 145.415 50.00625) (end 144.2075 48.79875) (width 0.2) (layer "F.Cu") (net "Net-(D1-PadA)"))
 (segment (start 141.44625 49.02) (end 141.44625 59.852606) (width 0.2) (layer "F.Cu") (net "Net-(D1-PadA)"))
 (segment (start 141.6675 48.79875) (end 141.44625 49.02) (width 0.2) (layer "F.Cu") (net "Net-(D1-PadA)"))
 (segment (start 144.2075 48.79875) (end 141.6675 48.79875) (width 0.2) (layer "F.Cu") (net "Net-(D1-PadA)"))
 (segment (start 187.0075 56.201356) (end 183.35625 59.852606) (width 0.2) (layer "F.Cu") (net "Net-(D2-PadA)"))
 (segment (start 187.0075 50.327606) (end 187.0075 56.201356) (width 0.2) (layer "F.Cu") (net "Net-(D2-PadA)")))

